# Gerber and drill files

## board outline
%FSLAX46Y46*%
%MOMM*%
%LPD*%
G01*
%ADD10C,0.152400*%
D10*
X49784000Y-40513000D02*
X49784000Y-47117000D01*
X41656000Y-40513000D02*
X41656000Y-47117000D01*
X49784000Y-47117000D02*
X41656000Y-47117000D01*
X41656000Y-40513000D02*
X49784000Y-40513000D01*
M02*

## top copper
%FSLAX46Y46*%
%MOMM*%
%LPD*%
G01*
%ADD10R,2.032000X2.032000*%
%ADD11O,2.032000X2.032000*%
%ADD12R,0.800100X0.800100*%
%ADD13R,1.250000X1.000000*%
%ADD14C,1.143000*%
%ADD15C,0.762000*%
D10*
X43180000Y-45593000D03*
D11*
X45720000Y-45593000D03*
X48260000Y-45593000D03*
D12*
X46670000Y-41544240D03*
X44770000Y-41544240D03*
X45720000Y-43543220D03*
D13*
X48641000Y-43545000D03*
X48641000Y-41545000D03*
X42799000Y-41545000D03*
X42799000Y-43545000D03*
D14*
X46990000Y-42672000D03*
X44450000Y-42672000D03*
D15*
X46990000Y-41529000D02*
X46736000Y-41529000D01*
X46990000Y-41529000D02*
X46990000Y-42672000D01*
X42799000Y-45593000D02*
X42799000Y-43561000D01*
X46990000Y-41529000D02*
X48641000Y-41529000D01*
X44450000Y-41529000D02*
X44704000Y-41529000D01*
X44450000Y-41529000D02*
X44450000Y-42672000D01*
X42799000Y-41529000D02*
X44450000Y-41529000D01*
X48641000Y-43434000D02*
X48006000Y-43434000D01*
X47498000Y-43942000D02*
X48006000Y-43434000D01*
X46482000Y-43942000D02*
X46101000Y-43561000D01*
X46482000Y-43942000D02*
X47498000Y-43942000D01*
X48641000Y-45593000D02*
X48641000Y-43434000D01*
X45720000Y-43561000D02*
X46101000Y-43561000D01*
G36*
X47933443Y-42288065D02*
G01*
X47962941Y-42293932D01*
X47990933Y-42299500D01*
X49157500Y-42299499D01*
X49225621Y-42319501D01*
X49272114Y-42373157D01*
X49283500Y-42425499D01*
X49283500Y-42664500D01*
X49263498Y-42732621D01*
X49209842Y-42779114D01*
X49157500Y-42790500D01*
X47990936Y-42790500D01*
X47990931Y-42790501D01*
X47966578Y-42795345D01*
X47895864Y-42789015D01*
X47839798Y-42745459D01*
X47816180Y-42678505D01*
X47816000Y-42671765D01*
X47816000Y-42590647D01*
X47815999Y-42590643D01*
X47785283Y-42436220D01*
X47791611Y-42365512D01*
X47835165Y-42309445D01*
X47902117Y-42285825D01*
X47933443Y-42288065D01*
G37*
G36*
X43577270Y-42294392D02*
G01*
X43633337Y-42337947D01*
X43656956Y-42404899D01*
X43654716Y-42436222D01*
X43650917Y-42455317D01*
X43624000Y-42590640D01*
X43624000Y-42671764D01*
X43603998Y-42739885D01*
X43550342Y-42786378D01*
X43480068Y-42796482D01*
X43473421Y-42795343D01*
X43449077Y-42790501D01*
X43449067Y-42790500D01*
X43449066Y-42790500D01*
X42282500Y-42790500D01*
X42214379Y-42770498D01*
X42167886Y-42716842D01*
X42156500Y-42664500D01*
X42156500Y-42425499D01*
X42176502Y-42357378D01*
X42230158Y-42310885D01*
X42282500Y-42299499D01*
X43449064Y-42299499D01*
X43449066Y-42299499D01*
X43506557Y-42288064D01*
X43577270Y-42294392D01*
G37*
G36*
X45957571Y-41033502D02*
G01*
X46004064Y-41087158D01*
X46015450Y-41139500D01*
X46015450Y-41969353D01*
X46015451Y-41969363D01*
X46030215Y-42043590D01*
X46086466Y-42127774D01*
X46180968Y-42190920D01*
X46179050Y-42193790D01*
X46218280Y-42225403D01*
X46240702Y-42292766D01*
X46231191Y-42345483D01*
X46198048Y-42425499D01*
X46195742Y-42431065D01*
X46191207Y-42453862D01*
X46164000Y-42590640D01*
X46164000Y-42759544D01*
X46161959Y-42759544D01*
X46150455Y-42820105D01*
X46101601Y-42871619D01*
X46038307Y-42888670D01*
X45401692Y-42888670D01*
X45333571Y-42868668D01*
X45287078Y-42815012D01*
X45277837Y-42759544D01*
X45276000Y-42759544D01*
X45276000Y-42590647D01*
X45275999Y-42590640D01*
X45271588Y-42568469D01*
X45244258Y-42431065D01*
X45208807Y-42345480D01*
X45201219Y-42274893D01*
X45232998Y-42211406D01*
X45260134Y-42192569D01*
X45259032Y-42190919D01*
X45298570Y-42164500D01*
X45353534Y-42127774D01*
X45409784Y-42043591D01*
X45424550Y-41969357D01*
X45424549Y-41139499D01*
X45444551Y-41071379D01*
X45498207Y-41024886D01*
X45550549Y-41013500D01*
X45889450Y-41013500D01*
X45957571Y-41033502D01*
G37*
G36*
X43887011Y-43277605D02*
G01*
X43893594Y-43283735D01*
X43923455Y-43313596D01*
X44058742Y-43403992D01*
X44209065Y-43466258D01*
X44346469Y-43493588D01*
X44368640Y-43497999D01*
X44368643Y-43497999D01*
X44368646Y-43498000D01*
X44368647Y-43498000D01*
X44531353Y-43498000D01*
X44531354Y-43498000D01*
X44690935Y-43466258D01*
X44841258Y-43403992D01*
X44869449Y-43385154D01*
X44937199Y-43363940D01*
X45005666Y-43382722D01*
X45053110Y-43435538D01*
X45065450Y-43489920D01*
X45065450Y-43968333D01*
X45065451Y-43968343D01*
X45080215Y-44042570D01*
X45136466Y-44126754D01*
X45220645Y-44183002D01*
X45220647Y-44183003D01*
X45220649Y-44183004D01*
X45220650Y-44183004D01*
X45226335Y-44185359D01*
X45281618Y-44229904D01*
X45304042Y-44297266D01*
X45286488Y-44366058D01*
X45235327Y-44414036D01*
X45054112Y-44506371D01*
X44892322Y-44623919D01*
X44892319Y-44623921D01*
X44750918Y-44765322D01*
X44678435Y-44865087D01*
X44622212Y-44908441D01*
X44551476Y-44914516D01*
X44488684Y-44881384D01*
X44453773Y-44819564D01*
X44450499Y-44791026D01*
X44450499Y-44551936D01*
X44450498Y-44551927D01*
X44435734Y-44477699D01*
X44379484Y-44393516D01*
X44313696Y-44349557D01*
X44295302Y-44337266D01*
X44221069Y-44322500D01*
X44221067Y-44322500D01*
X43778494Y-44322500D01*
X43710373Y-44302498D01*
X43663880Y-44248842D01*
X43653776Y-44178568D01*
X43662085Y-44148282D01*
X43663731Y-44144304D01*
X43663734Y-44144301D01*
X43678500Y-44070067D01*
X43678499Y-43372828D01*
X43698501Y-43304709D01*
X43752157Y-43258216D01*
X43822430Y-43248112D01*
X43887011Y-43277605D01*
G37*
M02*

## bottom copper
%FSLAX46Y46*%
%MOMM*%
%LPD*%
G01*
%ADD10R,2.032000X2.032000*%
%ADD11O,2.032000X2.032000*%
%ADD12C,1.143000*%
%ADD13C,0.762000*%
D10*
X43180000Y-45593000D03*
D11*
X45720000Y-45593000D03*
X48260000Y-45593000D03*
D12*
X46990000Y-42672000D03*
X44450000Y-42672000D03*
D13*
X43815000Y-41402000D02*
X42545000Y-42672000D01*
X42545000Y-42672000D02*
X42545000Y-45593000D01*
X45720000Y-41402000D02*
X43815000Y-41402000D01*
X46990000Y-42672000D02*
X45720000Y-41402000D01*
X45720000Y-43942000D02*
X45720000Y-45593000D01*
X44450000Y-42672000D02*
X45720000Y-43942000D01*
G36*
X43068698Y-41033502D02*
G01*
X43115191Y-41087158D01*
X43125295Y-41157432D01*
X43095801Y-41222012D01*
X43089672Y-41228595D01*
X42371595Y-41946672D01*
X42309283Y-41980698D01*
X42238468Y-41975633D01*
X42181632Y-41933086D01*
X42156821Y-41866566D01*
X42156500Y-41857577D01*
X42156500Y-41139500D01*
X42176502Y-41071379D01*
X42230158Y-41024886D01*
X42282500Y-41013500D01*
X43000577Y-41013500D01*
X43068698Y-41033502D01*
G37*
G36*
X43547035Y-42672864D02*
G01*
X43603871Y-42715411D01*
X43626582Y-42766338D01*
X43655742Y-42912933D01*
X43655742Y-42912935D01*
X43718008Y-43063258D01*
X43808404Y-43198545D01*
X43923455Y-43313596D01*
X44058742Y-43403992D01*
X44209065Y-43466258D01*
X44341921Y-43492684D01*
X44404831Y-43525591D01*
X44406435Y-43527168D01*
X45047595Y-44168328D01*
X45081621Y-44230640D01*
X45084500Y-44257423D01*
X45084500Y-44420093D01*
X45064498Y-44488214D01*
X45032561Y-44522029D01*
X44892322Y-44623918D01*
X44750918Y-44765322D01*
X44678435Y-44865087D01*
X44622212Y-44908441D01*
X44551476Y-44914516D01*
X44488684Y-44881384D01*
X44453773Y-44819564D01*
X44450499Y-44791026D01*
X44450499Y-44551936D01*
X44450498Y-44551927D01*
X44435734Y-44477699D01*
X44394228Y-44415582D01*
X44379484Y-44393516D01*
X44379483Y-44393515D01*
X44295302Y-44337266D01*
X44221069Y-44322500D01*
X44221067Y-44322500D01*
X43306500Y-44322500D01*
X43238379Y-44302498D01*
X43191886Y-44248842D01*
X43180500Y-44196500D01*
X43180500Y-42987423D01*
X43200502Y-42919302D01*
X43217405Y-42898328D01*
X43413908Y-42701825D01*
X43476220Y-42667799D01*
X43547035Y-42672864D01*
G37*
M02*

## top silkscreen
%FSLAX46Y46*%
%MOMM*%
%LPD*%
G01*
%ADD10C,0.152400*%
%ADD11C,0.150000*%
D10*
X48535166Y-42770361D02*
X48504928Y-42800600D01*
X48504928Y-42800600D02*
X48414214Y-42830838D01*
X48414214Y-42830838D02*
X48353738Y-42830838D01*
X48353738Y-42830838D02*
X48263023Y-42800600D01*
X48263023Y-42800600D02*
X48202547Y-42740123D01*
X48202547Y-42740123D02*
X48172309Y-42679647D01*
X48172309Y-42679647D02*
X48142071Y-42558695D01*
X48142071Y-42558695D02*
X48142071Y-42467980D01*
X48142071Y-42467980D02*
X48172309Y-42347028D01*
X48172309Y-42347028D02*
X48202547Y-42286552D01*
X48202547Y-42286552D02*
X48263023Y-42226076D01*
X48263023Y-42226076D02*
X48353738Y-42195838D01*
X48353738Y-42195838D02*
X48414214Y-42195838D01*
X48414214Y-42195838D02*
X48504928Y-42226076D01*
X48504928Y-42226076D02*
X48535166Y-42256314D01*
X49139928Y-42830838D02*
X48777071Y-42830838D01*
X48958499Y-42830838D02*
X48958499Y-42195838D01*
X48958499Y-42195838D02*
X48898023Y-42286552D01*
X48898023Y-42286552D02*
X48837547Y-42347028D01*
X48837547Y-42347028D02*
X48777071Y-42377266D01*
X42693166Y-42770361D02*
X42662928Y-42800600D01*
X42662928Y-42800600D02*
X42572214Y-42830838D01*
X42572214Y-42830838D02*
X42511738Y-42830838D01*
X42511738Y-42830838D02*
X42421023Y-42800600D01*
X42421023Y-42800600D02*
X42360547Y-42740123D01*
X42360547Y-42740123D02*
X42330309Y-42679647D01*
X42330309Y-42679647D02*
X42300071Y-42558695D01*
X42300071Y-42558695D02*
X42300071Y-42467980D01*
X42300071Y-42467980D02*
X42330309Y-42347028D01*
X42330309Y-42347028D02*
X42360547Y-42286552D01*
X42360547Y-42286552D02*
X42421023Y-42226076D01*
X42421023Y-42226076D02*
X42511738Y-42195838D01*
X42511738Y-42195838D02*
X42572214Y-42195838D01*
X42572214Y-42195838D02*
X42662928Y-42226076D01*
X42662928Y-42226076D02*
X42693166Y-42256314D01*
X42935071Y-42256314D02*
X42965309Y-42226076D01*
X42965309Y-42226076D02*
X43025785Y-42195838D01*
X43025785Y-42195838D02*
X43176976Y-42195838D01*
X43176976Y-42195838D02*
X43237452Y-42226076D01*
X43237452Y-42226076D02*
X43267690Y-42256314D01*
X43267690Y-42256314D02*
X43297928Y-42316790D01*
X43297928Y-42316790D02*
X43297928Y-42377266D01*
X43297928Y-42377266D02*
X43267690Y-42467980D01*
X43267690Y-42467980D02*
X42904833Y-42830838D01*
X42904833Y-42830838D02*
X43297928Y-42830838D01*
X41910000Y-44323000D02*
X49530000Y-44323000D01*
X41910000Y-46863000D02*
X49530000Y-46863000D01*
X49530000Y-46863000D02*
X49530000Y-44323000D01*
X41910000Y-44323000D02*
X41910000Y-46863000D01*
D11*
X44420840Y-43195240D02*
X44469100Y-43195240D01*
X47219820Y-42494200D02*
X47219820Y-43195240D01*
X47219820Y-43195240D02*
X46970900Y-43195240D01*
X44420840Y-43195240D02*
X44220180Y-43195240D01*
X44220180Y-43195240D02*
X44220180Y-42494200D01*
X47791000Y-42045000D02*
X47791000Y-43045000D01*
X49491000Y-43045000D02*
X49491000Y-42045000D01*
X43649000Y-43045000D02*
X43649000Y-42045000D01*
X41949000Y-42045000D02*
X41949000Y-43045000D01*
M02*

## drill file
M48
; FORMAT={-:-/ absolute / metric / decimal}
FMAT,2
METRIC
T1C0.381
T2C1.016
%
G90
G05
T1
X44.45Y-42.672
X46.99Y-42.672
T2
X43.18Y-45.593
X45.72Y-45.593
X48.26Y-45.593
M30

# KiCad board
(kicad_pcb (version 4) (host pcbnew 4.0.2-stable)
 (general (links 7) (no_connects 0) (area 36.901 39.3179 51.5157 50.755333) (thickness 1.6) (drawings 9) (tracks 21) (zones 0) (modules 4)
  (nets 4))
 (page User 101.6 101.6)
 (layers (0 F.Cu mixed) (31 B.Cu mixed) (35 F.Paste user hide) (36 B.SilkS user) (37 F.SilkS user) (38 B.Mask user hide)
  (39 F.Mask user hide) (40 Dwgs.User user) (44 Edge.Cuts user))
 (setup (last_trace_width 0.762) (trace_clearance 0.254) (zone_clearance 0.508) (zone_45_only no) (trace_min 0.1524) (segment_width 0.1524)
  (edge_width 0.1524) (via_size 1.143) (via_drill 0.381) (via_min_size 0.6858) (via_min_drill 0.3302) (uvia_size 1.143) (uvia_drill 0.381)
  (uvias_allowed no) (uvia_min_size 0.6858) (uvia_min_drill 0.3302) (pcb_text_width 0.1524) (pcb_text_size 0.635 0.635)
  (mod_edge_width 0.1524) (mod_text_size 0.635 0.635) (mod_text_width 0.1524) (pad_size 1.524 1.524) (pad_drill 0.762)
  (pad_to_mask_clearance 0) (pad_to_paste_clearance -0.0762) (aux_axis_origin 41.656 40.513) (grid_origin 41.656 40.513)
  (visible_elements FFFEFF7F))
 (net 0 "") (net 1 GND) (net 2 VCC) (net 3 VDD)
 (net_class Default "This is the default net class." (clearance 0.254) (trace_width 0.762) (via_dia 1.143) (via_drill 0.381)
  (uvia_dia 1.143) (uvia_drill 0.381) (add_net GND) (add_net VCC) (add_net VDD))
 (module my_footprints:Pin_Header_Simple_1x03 (layer F.Cu) (at 43.18 45.593 90)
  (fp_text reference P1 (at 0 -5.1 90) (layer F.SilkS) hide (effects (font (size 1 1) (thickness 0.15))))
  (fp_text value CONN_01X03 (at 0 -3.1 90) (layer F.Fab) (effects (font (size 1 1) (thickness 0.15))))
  (fp_line (start 1.27 -1.27) (end 1.27 6.35) (layer F.SilkS) (width 0.1524))
  (fp_line (start -1.27 -1.27) (end -1.27 6.35) (layer F.SilkS) (width 0.1524))
  (fp_line (start -1.27 6.35) (end 1.27 6.35) (layer F.SilkS) (width 0.1524))
  (fp_line (start 1.27 -1.27) (end -1.27 -1.27) (layer F.SilkS) (width 0.1524))
  (pad 1 thru_hole rect (at 0 0 90) (size 2.032 2.032) (drill 1.016) (layers *.Cu *.Mask) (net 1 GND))
  (pad 2 thru_hole oval (at 0 2.54 90) (size 2.032 2.032) (drill 1.016) (layers *.Cu *.Mask) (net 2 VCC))
  (pad 3 thru_hole oval (at 0 5.08 90) (size 2.032 2.032) (drill 1.016) (layers *.Cu *.Mask) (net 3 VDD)))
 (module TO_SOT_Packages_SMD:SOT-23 (layer F.Cu) (at 45.72 42.545 180)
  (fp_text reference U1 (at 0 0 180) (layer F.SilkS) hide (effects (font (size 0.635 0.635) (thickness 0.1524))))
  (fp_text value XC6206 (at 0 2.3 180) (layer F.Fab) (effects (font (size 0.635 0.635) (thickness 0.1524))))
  (fp_line (start 1.29916 -0.65024) (end 1.2509 -0.65024) (layer F.SilkS) (width 0.15))
  (fp_line (start -1.49982 0.0508) (end -1.49982 -0.65024) (layer F.SilkS) (width 0.15))
  (fp_line (start -1.49982 -0.65024) (end -1.2509 -0.65024) (layer F.SilkS) (width 0.15))
  (fp_line (start 1.29916 -0.65024) (end 1.49982 -0.65024) (layer F.SilkS) (width 0.15))
  (fp_line (start 1.49982 -0.65024) (end 1.49982 0.0508) (layer F.SilkS) (width 0.15))
  (pad 1 smd rect (at -0.95 1.00076 180) (size 0.8001 0.8001) (layers F.Cu F.Paste F.Mask) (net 1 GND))
  (pad 2 smd rect (at 0.95 1.00076 180) (size 0.8001 0.8001) (layers F.Cu F.Paste F.Mask) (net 2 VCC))
  (pad 3 smd rect (at 0 -0.99822 180) (size 0.8001 0.8001) (layers F.Cu F.Paste F.Mask) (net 3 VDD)))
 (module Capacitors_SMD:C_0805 (layer F.Cu) (at 48.641 42.545 90)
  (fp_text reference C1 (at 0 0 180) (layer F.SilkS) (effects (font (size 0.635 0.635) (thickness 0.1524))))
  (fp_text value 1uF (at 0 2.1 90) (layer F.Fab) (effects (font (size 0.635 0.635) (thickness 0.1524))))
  (fp_line (start 0.5 -0.85) (end -0.5 -0.85) (layer F.SilkS) (width 0.15))
  (fp_line (start -0.5 0.85) (end 0.5 0.85) (layer F.SilkS) (width 0.15))
  (pad 1 smd rect (at -1 0 90) (size 1 1.25) (layers F.Cu F.Paste F.Mask) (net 3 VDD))
  (pad 2 smd rect (at 1 0 90) (size 1 1.25) (layers F.Cu F.Paste F.Mask) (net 1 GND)))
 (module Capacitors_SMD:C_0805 (layer F.Cu) (at 42.799 42.545 270)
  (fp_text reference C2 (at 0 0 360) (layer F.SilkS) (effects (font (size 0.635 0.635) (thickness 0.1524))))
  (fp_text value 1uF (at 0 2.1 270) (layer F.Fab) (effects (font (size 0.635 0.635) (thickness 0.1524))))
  (fp_line (start 0.5 -0.85) (end -0.5 -0.85) (layer F.SilkS) (width 0.15))
  (fp_line (start -0.5 0.85) (end 0.5 0.85) (layer F.SilkS) (width 0.15))
  (pad 1 smd rect (at -1 0 270) (size 1 1.25) (layers F.Cu F.Paste F.Mask) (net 2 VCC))
  (pad 2 smd rect (at 1 0 270) (size 1 1.25) (layers F.Cu F.Paste F.Mask) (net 1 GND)))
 (gr_line (start 49.784 40.513) (end 49.784 47.117) (angle 90) (layer Edge.Cuts) (width 0.1524))
 (gr_line (start 41.656 40.513) (end 41.656 47.117) (angle 90) (layer Edge.Cuts) (width 0.1524))
 (gr_line (start 49.784 47.117) (end 41.656 47.117) (angle 90) (layer Edge.Cuts) (width 0.1524))
 (gr_line (start 41.656 40.513) (end 49.784 40.513) (angle 90) (layer Edge.Cuts) (width 0.1524))
 (segment (start 46.99 41.529) (end 46.736 41.529) (width 0.762) (layer F.Cu) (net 1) (status 30))
 (segment (start 43.815 41.402) (end 42.545 42.672) (width 0.762) (layer B.Cu) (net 1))
 (segment (start 46.99 41.529) (end 46.99 42.672) (width 0.762) (layer F.Cu) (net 1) (status 10))
 (segment (start 42.545 42.672) (end 42.545 45.593) (width 0.762) (layer B.Cu) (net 1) (status 20))
 (segment (start 45.72 41.402) (end 43.815 41.402) (width 0.762) (layer B.Cu) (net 1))
 (segment (start 46.99 42.672) (end 45.72 41.402) (width 0.762) (layer B.Cu) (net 1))
 (via (at 46.99 42.672) (size 1.143) (drill 0.381) (layers F.Cu B.Cu) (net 1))
 (segment (start 42.799 45.593) (end 42.799 43.561) (width 0.762) (layer F.Cu) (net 1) (status 30))
 (segment (start 46.99 41.529) (end 48.641 41.529) (width 0.762) (layer F.Cu) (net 1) (status 30))
 (segment (start 44.45 41.529) (end 44.704 41.529) (width 0.762) (layer F.Cu) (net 2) (status 30))
 (segment (start 44.45 41.529) (end 44.45 42.672) (width 0.762) (layer F.Cu) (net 2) (status 10))
 (segment (start 45.72 43.942) (end 45.72 45.593) (width 0.762) (layer B.Cu) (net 2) (status 20))
 (segment (start 44.45 42.672) (end 45.72 43.942) (width 0.762) (layer B.Cu) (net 2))
 (via (at 44.45 42.672) (size 1.143) (drill 0.381) (layers F.Cu B.Cu) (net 2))
 (segment (start 42.799 41.529) (end 44.45 41.529) (width 0.762) (layer F.Cu) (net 2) (status 30))
 (segment (start 48.641 43.434) (end 48.006 43.434) (width 0.762) (layer F.Cu) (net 3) (status 10))
 (segment (start 47.498 43.942) (end 48.006 43.434) (width 0.762) (layer F.Cu) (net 3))
 (segment (start 46.482 43.942) (end 46.101 43.561) (width 0.762) (layer F.Cu) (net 3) (status 20))
 (segment (start 46.482 43.942) (end 47.498 43.942) (width 0.762) (layer F.Cu) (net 3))
 (segment (start 48.641 45.593) (end 48.641 43.434) (width 0.762) (layer F.Cu) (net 3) (status 30))
 (segment (start 45.72 43.561) (end 46.101 43.561) (width 0.762) (layer F.Cu) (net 3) (status 30))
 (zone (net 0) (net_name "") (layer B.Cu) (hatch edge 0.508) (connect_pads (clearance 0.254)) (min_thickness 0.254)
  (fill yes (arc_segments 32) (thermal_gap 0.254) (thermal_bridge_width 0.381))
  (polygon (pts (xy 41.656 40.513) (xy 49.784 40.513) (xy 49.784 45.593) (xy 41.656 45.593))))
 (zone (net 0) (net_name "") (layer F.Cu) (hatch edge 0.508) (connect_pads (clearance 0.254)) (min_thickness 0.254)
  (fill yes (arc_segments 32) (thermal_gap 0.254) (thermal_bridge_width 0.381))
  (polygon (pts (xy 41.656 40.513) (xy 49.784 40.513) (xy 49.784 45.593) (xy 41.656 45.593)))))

